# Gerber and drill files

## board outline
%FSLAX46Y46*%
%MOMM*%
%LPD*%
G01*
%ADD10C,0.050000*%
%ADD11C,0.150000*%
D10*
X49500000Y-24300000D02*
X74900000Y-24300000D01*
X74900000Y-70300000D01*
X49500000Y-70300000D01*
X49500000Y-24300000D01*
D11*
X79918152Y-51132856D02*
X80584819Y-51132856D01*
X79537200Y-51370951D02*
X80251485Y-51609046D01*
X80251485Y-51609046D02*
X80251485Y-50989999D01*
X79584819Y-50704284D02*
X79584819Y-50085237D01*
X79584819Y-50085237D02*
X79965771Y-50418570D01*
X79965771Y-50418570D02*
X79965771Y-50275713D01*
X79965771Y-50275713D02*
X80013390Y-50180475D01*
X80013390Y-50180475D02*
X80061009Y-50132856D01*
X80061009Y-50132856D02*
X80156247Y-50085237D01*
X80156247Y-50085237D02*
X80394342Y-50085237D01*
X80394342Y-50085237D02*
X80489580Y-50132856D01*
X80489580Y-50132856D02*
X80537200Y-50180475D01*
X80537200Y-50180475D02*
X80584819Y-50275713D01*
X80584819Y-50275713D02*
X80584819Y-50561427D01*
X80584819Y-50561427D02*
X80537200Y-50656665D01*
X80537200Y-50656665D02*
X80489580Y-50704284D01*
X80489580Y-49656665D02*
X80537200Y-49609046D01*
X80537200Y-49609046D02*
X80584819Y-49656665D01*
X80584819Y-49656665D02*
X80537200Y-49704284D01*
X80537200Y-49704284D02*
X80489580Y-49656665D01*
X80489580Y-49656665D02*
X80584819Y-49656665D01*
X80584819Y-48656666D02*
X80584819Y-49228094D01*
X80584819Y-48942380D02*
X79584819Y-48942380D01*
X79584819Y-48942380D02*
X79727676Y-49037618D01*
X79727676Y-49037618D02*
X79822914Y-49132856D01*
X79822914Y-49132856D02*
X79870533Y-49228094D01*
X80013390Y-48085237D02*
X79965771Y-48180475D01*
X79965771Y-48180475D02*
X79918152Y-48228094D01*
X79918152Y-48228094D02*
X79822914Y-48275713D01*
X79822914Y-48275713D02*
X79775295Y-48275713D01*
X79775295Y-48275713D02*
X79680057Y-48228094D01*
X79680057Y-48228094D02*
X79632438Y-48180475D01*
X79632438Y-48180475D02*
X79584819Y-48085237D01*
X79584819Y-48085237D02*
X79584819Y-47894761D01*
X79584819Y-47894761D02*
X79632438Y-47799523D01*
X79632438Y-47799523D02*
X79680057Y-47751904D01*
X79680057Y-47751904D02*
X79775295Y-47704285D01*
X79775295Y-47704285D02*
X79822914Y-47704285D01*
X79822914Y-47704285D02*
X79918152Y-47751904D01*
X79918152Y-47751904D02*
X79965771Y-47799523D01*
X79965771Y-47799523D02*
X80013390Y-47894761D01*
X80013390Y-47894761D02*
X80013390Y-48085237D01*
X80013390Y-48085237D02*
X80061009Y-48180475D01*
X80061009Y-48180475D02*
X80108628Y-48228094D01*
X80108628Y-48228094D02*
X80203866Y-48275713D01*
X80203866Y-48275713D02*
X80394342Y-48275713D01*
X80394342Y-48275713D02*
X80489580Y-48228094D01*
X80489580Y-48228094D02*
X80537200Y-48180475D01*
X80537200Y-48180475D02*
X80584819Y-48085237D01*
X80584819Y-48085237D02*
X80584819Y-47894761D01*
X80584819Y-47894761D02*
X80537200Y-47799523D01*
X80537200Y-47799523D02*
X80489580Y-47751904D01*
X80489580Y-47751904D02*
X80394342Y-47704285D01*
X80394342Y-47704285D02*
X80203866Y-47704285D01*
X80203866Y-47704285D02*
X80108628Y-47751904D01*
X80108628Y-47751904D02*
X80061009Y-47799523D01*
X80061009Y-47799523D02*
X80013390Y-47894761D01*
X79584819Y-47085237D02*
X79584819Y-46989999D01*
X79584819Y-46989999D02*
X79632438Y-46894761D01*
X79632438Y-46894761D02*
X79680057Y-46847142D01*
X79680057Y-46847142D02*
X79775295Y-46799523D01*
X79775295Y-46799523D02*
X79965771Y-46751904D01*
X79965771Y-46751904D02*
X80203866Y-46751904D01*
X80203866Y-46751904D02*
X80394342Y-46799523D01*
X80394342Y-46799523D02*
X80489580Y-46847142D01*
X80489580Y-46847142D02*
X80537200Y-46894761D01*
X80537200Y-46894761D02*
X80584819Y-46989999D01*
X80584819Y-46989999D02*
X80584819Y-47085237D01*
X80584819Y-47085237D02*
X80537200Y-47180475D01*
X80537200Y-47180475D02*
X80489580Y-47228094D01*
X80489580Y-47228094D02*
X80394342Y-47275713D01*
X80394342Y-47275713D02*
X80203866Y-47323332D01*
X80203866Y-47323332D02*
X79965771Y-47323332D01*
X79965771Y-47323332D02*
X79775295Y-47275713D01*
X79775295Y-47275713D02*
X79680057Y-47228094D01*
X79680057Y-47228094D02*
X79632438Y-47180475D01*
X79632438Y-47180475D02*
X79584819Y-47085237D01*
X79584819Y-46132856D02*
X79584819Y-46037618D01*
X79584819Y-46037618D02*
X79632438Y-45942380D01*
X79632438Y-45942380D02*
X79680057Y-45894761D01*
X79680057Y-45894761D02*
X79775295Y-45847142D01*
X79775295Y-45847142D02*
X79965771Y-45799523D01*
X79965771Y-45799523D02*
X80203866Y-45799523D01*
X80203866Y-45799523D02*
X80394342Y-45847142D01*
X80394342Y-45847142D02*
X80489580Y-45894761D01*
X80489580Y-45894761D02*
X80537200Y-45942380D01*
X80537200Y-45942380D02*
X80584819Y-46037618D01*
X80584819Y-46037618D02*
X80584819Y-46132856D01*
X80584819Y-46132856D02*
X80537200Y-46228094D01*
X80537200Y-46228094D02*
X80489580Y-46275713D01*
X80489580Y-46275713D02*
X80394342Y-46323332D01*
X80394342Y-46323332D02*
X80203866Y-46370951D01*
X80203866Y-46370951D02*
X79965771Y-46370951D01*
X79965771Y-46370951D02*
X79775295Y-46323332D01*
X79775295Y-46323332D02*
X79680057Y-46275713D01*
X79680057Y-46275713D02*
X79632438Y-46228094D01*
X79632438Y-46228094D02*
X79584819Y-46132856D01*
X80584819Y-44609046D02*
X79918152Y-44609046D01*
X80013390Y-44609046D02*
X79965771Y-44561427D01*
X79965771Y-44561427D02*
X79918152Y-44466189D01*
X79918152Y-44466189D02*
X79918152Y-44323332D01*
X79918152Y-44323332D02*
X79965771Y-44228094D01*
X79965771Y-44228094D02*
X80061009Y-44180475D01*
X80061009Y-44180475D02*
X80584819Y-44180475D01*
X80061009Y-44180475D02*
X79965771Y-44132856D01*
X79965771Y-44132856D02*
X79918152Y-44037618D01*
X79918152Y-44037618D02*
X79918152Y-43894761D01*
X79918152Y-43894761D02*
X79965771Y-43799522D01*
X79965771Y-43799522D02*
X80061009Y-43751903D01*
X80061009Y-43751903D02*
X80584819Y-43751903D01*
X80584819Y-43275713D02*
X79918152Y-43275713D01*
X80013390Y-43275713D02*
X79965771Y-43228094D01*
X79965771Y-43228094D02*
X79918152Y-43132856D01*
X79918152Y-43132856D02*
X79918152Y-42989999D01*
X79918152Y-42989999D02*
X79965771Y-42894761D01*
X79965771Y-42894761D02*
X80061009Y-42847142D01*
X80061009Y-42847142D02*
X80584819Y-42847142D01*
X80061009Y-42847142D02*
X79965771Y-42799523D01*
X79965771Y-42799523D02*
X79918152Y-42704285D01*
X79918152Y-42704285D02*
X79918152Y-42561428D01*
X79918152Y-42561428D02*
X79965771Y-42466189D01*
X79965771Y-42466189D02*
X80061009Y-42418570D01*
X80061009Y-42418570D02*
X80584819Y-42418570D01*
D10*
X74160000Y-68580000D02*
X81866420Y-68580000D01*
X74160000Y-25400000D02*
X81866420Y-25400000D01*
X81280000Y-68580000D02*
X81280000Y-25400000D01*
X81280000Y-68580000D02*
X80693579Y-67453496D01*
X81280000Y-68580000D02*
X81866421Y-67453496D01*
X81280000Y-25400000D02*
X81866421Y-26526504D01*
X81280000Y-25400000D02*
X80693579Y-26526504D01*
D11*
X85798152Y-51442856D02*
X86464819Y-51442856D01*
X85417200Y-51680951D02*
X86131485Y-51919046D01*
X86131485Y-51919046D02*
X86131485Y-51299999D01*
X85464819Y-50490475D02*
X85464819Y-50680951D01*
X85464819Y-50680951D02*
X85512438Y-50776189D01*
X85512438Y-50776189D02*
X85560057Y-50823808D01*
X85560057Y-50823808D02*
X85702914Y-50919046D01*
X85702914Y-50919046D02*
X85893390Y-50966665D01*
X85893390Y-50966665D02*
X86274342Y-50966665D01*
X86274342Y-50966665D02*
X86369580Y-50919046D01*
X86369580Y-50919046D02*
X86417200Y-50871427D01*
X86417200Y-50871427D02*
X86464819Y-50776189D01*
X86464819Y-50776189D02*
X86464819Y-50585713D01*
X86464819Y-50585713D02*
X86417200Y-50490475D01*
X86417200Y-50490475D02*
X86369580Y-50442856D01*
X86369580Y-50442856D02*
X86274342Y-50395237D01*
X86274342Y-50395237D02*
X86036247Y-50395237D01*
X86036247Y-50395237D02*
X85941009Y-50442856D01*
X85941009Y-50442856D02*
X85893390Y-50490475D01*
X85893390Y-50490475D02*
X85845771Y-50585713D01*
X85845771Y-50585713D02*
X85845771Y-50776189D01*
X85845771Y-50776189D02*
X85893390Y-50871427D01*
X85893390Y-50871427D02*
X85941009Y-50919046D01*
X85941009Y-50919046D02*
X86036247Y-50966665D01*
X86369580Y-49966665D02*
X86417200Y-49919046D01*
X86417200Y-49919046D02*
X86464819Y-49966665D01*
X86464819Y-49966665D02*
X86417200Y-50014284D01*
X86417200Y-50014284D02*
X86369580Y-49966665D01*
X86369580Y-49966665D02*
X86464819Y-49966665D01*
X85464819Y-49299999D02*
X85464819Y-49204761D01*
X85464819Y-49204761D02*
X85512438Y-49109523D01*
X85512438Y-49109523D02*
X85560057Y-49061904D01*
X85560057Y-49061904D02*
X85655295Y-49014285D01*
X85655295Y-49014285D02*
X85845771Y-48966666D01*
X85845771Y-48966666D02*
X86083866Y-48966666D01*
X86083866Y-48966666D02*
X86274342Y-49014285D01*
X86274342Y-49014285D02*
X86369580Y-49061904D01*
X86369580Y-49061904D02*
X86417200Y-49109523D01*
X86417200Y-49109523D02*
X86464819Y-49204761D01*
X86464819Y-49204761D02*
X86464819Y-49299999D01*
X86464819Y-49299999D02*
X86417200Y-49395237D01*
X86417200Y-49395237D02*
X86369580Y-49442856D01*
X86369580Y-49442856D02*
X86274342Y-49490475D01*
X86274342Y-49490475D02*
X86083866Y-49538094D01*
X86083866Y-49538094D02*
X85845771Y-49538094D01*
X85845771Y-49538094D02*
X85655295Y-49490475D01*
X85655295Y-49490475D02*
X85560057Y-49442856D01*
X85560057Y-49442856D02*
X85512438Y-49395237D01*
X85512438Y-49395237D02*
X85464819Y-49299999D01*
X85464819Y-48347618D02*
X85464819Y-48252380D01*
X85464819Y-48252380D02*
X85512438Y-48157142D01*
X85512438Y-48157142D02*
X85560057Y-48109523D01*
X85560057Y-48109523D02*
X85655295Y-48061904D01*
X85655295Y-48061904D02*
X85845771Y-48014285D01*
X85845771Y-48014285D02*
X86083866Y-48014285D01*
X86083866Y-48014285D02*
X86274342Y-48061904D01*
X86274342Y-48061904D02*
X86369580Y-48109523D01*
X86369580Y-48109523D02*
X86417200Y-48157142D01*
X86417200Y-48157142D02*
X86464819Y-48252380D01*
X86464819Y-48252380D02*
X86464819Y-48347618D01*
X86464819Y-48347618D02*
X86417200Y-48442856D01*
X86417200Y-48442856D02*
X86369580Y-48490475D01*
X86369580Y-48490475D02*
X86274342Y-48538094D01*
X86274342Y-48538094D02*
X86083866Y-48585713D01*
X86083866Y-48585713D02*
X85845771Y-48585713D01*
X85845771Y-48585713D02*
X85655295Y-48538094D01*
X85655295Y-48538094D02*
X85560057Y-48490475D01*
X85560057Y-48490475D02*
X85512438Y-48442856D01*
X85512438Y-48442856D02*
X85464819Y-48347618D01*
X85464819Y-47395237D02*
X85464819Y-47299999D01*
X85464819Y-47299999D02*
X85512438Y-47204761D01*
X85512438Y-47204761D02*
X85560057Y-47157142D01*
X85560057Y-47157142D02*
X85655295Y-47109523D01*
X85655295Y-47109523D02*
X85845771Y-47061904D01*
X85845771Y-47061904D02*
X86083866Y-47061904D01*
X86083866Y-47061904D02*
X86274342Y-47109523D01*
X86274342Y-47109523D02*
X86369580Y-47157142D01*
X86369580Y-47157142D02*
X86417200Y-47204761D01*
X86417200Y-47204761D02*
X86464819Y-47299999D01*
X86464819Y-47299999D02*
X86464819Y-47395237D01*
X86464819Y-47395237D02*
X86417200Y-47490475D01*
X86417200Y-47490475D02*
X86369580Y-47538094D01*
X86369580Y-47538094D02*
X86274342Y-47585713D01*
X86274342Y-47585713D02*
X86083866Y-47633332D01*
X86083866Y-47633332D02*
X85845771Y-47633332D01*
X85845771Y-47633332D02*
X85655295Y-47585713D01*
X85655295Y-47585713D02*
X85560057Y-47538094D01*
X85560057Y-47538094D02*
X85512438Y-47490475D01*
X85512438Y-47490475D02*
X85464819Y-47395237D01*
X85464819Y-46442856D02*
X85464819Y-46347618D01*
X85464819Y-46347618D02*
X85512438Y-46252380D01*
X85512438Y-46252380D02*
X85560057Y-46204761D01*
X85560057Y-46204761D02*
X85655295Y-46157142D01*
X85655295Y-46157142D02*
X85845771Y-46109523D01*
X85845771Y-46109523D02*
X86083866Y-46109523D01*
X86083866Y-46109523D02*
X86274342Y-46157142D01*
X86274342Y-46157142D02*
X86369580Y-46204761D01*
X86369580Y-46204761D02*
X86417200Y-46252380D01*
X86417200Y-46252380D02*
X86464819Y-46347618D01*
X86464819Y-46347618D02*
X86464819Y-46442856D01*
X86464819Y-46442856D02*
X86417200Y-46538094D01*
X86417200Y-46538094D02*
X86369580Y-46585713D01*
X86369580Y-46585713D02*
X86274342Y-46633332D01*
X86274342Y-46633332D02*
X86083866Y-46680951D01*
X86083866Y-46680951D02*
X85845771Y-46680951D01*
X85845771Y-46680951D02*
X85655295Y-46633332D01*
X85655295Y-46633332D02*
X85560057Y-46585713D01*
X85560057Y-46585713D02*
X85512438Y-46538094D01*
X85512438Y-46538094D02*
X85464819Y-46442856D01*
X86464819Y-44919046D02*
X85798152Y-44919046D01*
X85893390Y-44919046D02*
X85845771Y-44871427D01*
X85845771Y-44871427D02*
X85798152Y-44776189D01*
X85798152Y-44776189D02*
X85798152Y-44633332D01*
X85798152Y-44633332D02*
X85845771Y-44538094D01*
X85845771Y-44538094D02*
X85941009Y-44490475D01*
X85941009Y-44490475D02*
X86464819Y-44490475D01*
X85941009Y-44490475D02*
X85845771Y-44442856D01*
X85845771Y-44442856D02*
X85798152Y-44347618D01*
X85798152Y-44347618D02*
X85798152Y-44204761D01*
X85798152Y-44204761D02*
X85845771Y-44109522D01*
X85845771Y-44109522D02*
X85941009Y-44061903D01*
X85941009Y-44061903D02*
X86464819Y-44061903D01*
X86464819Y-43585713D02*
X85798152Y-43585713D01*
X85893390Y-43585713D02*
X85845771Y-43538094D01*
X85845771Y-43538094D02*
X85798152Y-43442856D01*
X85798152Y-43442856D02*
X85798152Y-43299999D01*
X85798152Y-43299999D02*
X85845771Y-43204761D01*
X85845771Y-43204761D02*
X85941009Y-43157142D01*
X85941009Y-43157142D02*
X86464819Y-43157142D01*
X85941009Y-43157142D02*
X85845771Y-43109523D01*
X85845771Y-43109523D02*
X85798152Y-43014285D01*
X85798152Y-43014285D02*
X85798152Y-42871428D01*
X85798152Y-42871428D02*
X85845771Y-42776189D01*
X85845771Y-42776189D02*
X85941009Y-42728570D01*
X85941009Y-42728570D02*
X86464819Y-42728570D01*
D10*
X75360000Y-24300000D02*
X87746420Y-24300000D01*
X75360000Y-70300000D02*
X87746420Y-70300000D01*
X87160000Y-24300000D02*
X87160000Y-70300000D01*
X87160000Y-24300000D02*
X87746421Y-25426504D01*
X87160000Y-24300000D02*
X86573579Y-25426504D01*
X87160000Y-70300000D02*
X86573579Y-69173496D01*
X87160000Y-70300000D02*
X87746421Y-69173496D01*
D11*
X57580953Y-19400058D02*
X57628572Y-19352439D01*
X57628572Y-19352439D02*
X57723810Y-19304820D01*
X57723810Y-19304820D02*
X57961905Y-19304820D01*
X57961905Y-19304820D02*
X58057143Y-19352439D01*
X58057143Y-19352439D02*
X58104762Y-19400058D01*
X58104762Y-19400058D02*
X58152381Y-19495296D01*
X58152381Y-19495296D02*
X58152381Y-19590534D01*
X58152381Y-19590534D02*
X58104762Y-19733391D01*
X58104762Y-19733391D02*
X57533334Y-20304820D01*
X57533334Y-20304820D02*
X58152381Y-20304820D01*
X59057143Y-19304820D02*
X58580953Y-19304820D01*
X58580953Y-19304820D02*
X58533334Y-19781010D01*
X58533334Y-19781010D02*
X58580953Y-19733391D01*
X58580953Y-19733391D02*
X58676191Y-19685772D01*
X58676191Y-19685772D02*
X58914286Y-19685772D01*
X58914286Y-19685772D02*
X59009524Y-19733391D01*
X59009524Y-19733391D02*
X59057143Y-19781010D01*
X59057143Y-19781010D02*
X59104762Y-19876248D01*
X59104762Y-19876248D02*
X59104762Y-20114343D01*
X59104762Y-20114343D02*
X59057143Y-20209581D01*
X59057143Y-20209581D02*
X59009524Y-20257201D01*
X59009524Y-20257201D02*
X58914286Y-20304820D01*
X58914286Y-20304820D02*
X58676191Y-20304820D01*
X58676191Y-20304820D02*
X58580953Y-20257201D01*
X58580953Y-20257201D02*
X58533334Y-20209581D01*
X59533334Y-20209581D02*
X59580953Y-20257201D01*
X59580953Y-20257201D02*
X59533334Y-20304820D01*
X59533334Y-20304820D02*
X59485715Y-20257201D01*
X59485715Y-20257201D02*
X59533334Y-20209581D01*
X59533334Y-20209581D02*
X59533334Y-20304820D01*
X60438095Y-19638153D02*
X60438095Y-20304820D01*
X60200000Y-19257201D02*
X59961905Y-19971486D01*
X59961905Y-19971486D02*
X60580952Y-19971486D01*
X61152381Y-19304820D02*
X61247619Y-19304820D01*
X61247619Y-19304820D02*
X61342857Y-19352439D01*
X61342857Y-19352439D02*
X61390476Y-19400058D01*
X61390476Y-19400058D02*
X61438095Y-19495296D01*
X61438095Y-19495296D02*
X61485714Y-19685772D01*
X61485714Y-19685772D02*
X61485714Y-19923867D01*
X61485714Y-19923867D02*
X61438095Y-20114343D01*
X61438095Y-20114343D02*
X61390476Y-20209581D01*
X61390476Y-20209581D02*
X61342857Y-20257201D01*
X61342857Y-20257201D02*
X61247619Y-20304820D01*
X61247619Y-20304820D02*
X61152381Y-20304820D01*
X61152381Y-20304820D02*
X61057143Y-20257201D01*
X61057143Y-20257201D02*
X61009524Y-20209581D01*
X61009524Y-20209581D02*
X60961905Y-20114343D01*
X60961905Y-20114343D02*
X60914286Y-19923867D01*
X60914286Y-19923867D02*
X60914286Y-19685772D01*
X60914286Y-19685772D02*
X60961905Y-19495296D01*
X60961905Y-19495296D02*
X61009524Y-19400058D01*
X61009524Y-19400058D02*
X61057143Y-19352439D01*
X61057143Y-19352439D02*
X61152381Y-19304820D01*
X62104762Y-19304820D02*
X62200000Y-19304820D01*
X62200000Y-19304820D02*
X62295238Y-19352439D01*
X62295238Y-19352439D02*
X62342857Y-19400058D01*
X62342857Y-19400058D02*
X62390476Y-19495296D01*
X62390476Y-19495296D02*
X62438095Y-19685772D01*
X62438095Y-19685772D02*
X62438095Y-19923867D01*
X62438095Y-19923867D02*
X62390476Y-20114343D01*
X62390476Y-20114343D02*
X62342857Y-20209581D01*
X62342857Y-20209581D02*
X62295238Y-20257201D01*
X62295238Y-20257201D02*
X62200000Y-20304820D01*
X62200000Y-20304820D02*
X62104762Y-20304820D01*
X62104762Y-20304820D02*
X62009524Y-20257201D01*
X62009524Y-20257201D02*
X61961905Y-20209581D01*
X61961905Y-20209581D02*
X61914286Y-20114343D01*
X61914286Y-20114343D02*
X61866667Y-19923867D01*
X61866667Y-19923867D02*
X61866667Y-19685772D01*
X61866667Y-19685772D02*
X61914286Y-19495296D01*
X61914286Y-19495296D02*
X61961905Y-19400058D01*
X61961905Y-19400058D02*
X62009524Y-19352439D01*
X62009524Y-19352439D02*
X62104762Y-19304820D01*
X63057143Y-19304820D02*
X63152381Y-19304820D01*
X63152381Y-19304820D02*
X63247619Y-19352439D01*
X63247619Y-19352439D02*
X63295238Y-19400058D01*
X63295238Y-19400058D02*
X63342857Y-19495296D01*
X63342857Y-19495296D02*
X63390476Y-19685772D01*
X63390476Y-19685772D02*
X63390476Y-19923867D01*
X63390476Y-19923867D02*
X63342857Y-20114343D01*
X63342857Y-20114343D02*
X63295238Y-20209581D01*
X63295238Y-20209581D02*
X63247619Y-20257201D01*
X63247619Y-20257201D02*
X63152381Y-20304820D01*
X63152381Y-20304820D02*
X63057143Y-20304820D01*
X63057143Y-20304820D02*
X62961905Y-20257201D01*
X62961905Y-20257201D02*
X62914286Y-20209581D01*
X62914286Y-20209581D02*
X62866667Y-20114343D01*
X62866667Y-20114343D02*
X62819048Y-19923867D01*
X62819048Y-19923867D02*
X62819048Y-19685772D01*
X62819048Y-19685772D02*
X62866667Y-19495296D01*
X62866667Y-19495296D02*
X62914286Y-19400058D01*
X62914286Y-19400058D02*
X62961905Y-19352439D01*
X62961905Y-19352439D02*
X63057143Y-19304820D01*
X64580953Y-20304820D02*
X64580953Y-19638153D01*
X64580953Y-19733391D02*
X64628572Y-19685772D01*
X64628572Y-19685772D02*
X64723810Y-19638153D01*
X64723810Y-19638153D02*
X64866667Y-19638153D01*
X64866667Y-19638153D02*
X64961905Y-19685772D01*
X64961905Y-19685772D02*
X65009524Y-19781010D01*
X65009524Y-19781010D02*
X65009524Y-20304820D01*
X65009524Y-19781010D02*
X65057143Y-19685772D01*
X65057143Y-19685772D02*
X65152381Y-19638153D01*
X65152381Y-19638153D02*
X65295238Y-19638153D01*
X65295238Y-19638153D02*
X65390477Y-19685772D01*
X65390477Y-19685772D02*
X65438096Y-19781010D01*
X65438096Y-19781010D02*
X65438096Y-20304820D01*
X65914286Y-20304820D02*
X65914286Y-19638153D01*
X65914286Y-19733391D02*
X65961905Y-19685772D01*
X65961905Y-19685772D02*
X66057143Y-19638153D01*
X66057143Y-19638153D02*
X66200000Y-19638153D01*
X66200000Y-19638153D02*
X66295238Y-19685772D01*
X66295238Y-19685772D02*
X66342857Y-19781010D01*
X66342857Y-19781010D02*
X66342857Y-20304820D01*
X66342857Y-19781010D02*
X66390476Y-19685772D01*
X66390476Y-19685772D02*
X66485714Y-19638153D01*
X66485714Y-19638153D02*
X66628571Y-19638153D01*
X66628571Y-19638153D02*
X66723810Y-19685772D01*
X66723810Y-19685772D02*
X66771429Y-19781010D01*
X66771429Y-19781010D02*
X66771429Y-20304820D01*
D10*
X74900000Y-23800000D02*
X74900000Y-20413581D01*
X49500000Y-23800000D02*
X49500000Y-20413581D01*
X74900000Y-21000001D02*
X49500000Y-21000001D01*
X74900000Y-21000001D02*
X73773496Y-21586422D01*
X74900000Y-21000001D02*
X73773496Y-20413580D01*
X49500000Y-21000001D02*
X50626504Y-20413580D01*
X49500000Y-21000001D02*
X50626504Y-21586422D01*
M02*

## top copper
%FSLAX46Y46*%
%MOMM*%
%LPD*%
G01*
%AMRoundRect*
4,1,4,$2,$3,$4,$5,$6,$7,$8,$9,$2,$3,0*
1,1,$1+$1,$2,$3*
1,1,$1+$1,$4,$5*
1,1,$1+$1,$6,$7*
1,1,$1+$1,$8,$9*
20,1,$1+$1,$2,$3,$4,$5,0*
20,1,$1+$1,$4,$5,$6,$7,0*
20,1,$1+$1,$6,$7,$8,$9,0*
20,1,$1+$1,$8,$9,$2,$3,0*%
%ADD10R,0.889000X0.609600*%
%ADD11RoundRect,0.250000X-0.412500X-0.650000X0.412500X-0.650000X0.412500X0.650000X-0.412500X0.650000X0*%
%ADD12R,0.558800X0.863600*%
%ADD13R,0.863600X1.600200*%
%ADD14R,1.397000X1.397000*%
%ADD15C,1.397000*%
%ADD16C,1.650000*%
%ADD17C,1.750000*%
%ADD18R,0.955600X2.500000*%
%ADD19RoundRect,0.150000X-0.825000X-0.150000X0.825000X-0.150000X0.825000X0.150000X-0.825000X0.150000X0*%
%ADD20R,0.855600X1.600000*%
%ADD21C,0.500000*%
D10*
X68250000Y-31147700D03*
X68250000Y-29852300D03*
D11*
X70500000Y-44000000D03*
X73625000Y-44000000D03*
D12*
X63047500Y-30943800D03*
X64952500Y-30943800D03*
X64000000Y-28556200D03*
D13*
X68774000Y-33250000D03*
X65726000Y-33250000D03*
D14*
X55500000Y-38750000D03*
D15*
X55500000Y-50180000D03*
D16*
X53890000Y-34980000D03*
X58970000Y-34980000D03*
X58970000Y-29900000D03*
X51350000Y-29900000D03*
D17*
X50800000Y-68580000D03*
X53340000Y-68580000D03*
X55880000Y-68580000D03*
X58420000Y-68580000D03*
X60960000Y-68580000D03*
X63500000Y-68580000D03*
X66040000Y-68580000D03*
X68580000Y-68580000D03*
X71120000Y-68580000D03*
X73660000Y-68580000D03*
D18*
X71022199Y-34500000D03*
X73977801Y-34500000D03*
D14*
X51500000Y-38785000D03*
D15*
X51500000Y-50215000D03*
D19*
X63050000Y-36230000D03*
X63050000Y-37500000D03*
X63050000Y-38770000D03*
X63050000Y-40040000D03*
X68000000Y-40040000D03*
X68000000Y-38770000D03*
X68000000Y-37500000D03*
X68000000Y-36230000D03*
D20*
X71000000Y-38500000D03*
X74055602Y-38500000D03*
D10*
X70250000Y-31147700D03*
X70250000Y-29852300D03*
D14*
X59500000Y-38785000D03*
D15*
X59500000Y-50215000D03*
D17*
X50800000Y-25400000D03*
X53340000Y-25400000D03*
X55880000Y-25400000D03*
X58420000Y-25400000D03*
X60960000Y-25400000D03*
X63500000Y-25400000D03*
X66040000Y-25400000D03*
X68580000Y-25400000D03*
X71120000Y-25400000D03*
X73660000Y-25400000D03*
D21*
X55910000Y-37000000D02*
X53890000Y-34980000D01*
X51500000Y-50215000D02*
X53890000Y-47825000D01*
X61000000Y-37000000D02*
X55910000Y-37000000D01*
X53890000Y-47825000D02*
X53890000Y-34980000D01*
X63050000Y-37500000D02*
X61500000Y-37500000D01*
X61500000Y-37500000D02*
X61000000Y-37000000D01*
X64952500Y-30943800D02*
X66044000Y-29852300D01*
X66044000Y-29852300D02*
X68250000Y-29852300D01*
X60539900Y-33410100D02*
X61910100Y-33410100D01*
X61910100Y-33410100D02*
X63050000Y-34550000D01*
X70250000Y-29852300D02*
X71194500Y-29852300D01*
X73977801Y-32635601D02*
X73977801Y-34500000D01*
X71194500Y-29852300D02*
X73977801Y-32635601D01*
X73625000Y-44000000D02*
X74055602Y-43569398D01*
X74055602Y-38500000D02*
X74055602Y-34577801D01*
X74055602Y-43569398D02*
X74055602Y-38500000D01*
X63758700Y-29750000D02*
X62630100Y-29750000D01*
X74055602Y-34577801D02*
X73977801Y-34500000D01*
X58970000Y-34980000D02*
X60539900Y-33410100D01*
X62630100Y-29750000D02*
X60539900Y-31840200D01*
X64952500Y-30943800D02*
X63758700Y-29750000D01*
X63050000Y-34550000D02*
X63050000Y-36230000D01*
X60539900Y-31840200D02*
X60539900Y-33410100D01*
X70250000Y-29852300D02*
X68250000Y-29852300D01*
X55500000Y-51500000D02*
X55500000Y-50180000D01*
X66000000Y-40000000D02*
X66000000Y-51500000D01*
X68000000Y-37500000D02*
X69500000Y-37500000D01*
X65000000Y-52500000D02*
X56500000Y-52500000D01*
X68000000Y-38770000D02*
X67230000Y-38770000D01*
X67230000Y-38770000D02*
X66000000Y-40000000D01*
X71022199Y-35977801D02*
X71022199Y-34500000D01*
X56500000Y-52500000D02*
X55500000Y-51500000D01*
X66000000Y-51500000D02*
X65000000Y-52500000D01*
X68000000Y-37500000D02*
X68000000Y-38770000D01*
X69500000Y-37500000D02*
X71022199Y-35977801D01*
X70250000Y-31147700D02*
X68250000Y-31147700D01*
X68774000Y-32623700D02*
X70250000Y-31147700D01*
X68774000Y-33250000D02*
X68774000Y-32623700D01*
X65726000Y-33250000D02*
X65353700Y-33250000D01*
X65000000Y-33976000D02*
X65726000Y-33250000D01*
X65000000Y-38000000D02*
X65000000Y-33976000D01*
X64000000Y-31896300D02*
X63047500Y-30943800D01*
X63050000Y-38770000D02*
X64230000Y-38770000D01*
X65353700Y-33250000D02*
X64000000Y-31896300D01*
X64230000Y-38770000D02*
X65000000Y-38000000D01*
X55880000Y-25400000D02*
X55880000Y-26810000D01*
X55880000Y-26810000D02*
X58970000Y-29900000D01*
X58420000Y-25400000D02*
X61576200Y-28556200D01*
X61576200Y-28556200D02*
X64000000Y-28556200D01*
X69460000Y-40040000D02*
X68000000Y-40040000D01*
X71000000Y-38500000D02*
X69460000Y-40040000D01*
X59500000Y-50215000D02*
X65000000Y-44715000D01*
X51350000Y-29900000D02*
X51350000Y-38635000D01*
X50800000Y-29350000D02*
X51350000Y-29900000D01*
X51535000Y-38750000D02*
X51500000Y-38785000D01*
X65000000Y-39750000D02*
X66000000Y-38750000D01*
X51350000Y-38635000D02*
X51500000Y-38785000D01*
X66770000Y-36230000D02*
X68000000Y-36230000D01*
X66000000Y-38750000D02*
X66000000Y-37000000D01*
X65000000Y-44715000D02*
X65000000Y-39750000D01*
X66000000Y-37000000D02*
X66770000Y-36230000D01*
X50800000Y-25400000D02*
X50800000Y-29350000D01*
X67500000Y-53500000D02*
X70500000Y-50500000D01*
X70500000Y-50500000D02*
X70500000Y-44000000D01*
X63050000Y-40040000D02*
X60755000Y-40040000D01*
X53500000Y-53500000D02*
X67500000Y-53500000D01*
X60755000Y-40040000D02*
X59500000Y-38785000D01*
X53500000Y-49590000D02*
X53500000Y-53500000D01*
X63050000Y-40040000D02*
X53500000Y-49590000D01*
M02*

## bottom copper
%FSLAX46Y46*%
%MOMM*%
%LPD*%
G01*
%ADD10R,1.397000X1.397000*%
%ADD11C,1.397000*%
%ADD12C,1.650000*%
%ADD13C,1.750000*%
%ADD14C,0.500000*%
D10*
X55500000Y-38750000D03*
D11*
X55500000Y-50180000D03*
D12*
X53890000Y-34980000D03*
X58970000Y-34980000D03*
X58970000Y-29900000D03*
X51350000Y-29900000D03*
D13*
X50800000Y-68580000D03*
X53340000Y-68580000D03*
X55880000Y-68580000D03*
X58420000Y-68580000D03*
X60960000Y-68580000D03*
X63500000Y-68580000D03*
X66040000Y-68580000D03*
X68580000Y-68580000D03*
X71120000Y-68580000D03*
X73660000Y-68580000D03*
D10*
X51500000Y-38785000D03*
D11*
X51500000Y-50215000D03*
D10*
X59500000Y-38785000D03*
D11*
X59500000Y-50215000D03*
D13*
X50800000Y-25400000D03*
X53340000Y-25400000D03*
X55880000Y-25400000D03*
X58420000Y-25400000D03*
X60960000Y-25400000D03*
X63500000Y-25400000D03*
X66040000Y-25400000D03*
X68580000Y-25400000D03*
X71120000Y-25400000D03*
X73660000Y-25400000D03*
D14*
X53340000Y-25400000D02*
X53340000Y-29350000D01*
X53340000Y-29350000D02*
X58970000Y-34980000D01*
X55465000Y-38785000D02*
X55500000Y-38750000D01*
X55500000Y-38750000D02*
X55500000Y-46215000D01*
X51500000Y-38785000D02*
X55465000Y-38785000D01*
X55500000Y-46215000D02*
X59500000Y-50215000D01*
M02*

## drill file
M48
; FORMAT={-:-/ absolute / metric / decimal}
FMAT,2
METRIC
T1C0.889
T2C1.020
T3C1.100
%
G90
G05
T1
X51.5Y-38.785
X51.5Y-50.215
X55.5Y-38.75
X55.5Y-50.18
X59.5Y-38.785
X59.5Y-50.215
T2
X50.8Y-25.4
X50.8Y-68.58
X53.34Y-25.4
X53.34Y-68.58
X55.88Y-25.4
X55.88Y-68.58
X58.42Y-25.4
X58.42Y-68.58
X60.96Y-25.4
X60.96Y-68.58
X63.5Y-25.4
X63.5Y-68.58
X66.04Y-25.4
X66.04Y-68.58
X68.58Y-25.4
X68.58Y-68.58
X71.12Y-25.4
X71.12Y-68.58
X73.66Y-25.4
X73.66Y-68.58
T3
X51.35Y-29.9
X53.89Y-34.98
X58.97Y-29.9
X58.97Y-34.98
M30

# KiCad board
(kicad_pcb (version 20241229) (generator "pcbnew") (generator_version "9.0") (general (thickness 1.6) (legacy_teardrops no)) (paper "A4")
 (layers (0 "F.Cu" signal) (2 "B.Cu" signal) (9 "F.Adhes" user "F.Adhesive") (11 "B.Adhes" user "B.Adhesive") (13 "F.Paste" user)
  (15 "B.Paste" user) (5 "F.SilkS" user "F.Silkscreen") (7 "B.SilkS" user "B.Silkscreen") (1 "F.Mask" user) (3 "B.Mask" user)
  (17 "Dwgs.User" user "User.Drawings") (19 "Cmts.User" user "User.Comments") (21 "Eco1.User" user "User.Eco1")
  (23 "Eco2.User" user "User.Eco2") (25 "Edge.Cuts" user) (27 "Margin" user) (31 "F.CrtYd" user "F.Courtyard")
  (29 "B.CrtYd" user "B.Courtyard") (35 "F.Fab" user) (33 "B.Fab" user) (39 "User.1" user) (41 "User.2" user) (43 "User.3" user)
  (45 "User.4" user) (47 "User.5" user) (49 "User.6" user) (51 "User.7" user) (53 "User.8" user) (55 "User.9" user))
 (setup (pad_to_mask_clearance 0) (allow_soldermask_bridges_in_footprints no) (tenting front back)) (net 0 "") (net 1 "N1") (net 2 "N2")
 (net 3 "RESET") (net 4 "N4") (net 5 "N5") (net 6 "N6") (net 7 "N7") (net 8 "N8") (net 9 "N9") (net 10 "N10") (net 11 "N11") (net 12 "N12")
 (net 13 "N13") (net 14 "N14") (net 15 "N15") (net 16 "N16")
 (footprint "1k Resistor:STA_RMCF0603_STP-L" (layer "F.Cu") (at 68.25 30.5 90)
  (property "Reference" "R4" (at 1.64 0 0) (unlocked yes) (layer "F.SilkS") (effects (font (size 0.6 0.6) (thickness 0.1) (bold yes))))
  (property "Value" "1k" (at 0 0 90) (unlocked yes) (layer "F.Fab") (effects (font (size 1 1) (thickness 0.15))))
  (pad "1" smd rect (at -0.6477 0 90) (size 0.6096 0.889) (layers "F.Cu" "F.Mask" "F.Paste") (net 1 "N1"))
  (pad "2" smd rect (at 0.6477 0 90) (size 0.6096 0.889) (layers "F.Cu" "F.Mask" "F.Paste") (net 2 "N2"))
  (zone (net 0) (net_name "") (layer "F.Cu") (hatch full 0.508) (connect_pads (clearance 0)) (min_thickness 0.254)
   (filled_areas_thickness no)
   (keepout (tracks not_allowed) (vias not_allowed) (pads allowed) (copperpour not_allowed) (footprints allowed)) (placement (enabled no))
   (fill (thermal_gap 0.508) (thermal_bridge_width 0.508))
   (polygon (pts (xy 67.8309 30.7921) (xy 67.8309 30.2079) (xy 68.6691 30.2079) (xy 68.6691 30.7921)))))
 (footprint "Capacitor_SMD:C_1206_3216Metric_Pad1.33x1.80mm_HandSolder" (layer "F.Cu") (at 72.0625 44)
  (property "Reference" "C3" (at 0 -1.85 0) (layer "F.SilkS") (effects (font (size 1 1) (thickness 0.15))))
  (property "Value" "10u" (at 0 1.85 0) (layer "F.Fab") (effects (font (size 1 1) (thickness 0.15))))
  (pad "1" smd roundrect (at -1.5625 0) (size 1.325 1.8) (layers "F.Cu" "F.Mask" "F.Paste") (roundrect_rratio 0.188679) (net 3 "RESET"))
  (pad "2" smd roundrect (at 1.5625 0) (size 1.325 1.8) (layers "F.Cu" "F.Mask" "F.Paste") (roundrect_rratio 0.188679) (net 2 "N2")))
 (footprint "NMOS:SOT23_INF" (layer "F.Cu") (at 64 29.75)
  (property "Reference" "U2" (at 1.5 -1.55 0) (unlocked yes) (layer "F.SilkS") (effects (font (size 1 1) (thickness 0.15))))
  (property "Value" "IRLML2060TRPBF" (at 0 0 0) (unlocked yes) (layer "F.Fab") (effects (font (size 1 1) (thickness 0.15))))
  (pad "1" smd rect (at -0.9525 1.1938) (size 0.5588 0.8636) (layers "F.Cu" "F.Mask" "F.Paste") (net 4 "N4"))
  (pad "2" smd rect (at 0.9525 1.1938) (size 0.5588 0.8636) (layers "F.Cu" "F.Mask" "F.Paste") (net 2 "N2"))
  (pad "3" smd rect (at 0 -1.1938) (size 0.5588 0.8636) (layers "F.Cu" "F.Mask" "F.Paste") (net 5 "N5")))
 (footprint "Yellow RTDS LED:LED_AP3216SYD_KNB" (layer "F.Cu") (at 67.25 33.25 180)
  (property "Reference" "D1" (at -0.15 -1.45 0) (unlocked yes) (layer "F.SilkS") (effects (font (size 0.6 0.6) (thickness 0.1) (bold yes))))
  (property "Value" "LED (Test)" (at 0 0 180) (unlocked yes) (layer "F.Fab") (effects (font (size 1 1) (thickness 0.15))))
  (pad "1" smd rect (at -1.524 0 180) (size 0.8636 1.6002) (layers "F.Cu" "F.Mask" "F.Paste") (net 1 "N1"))
  (pad "2" smd rect (at 1.524 0 180) (size 0.8636 1.6002) (layers "F.Cu" "F.Mask" "F.Paste") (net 4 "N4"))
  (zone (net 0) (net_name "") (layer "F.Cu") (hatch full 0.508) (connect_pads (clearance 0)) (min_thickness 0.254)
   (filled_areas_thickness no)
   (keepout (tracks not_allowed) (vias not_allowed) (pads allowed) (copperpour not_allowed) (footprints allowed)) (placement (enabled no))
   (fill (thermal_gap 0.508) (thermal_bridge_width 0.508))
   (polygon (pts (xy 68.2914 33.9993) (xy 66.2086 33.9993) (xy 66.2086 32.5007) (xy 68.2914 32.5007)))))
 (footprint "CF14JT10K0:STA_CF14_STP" (layer "F.Cu") (at 55.5 38.75 -90)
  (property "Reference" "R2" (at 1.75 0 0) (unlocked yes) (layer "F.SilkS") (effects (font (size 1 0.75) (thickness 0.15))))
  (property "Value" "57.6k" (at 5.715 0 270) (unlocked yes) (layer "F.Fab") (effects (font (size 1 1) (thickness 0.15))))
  (pad "1" thru_hole rect (at 0 0 270) (size 1.397 1.397) (drill 0.889) (layers "*.Cu" "*.Mask") (remove_unused_layers no) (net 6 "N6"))
  (pad "2" thru_hole circle (at 11.43 0 270) (size 1.397 1.397) (drill 0.889) (layers "*.Cu" "*.Mask") (remove_unused_layers no)
   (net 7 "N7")))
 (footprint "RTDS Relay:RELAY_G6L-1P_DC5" (layer "F.Cu") (at 55.16 32.44)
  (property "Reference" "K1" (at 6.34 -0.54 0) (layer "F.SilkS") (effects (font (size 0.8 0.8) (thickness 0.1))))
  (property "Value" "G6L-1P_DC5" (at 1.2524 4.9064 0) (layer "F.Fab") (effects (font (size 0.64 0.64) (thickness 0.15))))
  (pad "2" thru_hole circle (at -1.27 2.54) (size 1.65 1.65) (drill 1.1) (layers "*.Cu" "*.Mask") (remove_unused_layers no) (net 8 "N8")
   (solder_mask_margin 0.102))
  (pad "4" thru_hole circle (at 3.81 2.54) (size 1.65 1.65) (drill 1.1) (layers "*.Cu" "*.Mask") (remove_unused_layers no) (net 2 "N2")
   (solder_mask_margin 0.102))
  (pad "5" thru_hole circle (at 3.81 -2.54) (size 1.65 1.65) (drill 1.1) (layers "*.Cu" "*.Mask") (remove_unused_layers no) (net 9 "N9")
   (solder_mask_margin 0.102))
  (pad "8" thru_hole circle (at -3.81 -2.54) (size 1.65 1.65) (drill 1.1) (layers "*.Cu" "*.Mask") (remove_unused_layers no) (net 6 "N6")
   (solder_mask_margin 0.102)))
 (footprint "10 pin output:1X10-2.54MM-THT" (layer "F.Cu") (at 50.8 68.58)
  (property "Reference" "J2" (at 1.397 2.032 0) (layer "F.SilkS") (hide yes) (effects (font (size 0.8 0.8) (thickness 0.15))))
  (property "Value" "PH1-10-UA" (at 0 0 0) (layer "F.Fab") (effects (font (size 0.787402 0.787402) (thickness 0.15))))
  (pad "1" thru_hole circle (at 0 0) (size 1.75 1.75) (drill 1.02) (layers "*.Cu" "*.Mask") (remove_unused_layers no)
   (solder_mask_margin 0.102))
  (pad "2" thru_hole circle (at 2.54 0) (size 1.75 1.75) (drill 1.02) (layers "*.Cu" "*.Mask") (remove_unused_layers no)
   (solder_mask_margin 0.102))
  (pad "3" thru_hole circle (at 5.08 0) (size 1.75 1.75) (drill 1.02) (layers "*.Cu" "*.Mask") (remove_unused_layers no)
   (solder_mask_margin 0.102))
  (pad "4" thru_hole circle (at 7.62 0) (size 1.75 1.75) (drill 1.02) (layers "*.Cu" "*.Mask") (remove_unused_layers no)
   (solder_mask_margin 0.102))
  (pad "5" thru_hole circle (at 10.16 0) (size 1.75 1.75) (drill 1.02) (layers "*.Cu" "*.Mask") (remove_unused_layers no)
   (solder_mask_margin 0.102))
  (pad "6" thru_hole circle (at 12.7 0) (size 1.75 1.75) (drill 1.02) (layers "*.Cu" "*.Mask") (remove_unused_layers no)
   (solder_mask_margin 0.102))
  (pad "7" thru_hole circle (at 15.24 0) (size 1.75 1.75) (drill 1.02) (layers "*.Cu" "*.Mask") (remove_unused_layers no)
   (solder_mask_margin 0.102))
  (pad "8" thru_hole circle (at 17.78 0) (size 1.75 1.75) (drill 1.02) (layers "*.Cu" "*.Mask") (remove_unused_layers no)
   (solder_mask_margin 0.102))
  (pad "9" thru_hole circle (at 20.32 0) (size 1.75 1.75) (drill 1.02) (layers "*.Cu" "*.Mask") (remove_unused_layers no)
   (solder_mask_margin 0.102))
  (pad "10" thru_hole circle (at 22.86 0) (size 1.75 1.75) (drill 1.02) (layers "*.Cu" "*.Mask") (remove_unused_layers no)
   (solder_mask_margin 0.102)))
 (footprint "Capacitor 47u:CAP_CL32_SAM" (layer "F.Cu") (at 72.5 34.5)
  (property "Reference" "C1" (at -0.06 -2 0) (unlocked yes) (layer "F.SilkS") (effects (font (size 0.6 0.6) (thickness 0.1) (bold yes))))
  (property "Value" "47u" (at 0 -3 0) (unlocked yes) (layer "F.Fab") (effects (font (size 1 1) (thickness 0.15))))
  (pad "1" smd rect (at -1.477801 0) (size 0.9556 2.5) (layers "F.Cu" "F.Mask" "F.Paste") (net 7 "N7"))
  (pad "2" smd rect (at 1.477801 0) (size 0.9556 2.5) (layers "F.Cu" "F.Mask" "F.Paste") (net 2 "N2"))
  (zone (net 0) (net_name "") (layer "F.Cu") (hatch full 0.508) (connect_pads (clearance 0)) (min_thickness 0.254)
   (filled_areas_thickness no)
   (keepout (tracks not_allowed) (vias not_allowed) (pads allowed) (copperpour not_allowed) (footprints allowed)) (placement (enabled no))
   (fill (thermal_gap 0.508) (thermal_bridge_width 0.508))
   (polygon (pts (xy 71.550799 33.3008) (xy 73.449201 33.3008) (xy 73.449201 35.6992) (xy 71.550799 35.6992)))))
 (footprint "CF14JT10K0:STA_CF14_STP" (layer "F.Cu") (at 51.5 38.785 -90)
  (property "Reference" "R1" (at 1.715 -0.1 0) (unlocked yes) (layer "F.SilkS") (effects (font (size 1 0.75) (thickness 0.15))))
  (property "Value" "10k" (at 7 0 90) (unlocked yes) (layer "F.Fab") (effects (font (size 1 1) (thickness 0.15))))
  (pad "1" thru_hole rect (at 0 0 270) (size 1.397 1.397) (drill 0.889) (layers "*.Cu" "*.Mask") (remove_unused_layers no) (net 6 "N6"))
  (pad "2" thru_hole circle (at 11.43 0 270) (size 1.397 1.397) (drill 0.889) (layers "*.Cu" "*.Mask") (remove_unused_layers no)
   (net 8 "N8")))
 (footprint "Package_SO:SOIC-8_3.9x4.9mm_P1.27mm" (layer "F.Cu") (at 65.525 38.135)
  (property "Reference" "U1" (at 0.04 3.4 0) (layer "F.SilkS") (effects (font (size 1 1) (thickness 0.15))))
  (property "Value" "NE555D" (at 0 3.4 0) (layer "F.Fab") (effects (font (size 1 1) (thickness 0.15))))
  (pad "1" smd roundrect (at -2.475 -1.905) (size 1.95 0.6) (layers "F.Cu" "F.Mask" "F.Paste") (roundrect_rratio 0.25) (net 2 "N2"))
  (pad "2" smd roundrect (at -2.475 -0.635) (size 1.95 0.6) (layers "F.Cu" "F.Mask" "F.Paste") (roundrect_rratio 0.25) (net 8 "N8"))
  (pad "3" smd roundrect (at -2.475 0.635) (size 1.95 0.6) (layers "F.Cu" "F.Mask" "F.Paste") (roundrect_rratio 0.25) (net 4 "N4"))
  (pad "4" smd roundrect (at -2.475 1.905) (size 1.95 0.6) (layers "F.Cu" "F.Mask" "F.Paste") (roundrect_rratio 0.25) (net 3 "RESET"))
  (pad "5" smd roundrect (at 2.475 1.905) (size 1.95 0.6) (layers "F.Cu" "F.Mask" "F.Paste") (roundrect_rratio 0.25) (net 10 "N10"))
  (pad "6" smd roundrect (at 2.475 0.635) (size 1.95 0.6) (layers "F.Cu" "F.Mask" "F.Paste") (roundrect_rratio 0.25) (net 7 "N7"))
  (pad "7" smd roundrect (at 2.475 -0.635) (size 1.95 0.6) (layers "F.Cu" "F.Mask" "F.Paste") (roundrect_rratio 0.25) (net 7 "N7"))
  (pad "8" smd roundrect (at 2.475 -1.905) (size 1.95 0.6) (layers "F.Cu" "F.Mask" "F.Paste") (roundrect_rratio 0.25) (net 6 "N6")))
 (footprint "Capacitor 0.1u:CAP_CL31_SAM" (layer "F.Cu") (at 72.527801 38.5)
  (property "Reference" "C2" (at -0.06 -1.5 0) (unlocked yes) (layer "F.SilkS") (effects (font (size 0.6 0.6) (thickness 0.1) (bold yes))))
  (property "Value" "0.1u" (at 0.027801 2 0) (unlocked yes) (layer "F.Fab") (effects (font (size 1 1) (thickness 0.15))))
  (pad "1" smd rect (at -1.527801 0) (size 0.8556 1.6) (layers "F.Cu" "F.Mask" "F.Paste") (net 10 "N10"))
  (pad "2" smd rect (at 1.527801 0) (size 0.8556 1.6) (layers "F.Cu" "F.Mask" "F.Paste") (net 2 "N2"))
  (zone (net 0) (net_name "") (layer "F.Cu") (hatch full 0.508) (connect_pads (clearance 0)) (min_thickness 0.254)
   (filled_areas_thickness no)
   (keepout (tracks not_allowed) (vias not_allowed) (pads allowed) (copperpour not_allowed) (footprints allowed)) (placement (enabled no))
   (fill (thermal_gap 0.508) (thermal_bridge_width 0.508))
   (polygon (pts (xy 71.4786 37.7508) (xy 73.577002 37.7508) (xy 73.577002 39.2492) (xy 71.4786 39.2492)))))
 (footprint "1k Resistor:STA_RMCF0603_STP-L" (layer "F.Cu") (at 70.25 30.5 90)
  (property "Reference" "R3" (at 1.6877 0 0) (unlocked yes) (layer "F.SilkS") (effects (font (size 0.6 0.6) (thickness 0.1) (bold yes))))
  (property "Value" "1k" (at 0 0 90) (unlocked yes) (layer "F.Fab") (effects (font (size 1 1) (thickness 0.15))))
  (pad "1" smd rect (at -0.6477 0 90) (size 0.6096 0.889) (layers "F.Cu" "F.Mask" "F.Paste") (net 1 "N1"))
  (pad "2" smd rect (at 0.6477 0 90) (size 0.6096 0.889) (layers "F.Cu" "F.Mask" "F.Paste") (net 2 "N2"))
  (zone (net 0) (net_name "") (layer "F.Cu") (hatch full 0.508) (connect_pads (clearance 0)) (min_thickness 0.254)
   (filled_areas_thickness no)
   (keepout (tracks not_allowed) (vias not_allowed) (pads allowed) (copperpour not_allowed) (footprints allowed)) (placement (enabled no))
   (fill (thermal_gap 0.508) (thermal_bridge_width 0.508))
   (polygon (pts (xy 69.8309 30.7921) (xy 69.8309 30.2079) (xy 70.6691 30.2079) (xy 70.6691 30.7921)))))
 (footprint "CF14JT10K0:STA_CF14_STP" (layer "F.Cu") (at 59.5 38.785 -90)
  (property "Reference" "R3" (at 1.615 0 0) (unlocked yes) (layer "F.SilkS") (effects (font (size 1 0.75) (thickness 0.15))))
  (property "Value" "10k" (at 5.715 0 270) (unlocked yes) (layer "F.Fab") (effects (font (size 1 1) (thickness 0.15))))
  (pad "1" thru_hole rect (at 0 0 270) (size 1.397 1.397) (drill 0.889) (layers "*.Cu" "*.Mask") (remove_unused_layers no) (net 3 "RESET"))
  (pad "2" thru_hole circle (at 11.43 0 270) (size 1.397 1.397) (drill 0.889) (layers "*.Cu" "*.Mask") (remove_unused_layers no)
   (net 6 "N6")))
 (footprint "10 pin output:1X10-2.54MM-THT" (layer "F.Cu") (at 50.8 25.4)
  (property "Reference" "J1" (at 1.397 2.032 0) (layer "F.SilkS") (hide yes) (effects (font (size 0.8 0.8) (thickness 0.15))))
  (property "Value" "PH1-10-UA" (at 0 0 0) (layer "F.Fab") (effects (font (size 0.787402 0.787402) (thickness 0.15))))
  (pad "1" thru_hole circle (at 0 0) (size 1.75 1.75) (drill 1.02) (layers "*.Cu" "*.Mask") (remove_unused_layers no) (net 6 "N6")
   (solder_mask_margin 0.102))
  (pad "2" thru_hole circle (at 2.54 0) (size 1.75 1.75) (drill 1.02) (layers "*.Cu" "*.Mask") (remove_unused_layers no) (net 2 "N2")
   (solder_mask_margin 0.102))
  (pad "3" thru_hole circle (at 5.08 0) (size 1.75 1.75) (drill 1.02) (layers "*.Cu" "*.Mask") (remove_unused_layers no) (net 9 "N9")
   (solder_mask_margin 0.102))
  (pad "4" thru_hole circle (at 7.62 0) (size 1.75 1.75) (drill 1.02) (layers "*.Cu" "*.Mask") (remove_unused_layers no) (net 5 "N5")
   (solder_mask_margin 0.102))
  (pad "5" thru_hole circle (at 10.16 0) (size 1.75 1.75) (drill 1.02) (layers "*.Cu" "*.Mask") (remove_unused_layers no) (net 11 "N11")
   (solder_mask_margin 0.102))
  (pad "6" thru_hole circle (at 12.7 0) (size 1.75 1.75) (drill 1.02) (layers "*.Cu" "*.Mask") (remove_unused_layers no) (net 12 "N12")
   (solder_mask_margin 0.102))
  (pad "7" thru_hole circle (at 15.24 0) (size 1.75 1.75) (drill 1.02) (layers "*.Cu" "*.Mask") (remove_unused_layers no) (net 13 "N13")
   (solder_mask_margin 0.102))
  (pad "8" thru_hole circle (at 17.78 0) (size 1.75 1.75) (drill 1.02) (layers "*.Cu" "*.Mask") (remove_unused_layers no) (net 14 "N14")
   (solder_mask_margin 0.102))
  (pad "9" thru_hole circle (at 20.32 0) (size 1.75 1.75) (drill 1.02) (layers "*.Cu" "*.Mask") (remove_unused_layers no) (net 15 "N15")
   (solder_mask_margin 0.102))
  (pad "10" thru_hole circle (at 22.86 0) (size 1.75 1.75) (drill 1.02) (layers "*.Cu" "*.Mask") (remove_unused_layers no) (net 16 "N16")
   (solder_mask_margin 0.102)))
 (gr_rect (start 49.5 24.3) (end 74.9 70.3) (stroke (width 0.05) (type default)) (fill no) (layer "Edge.Cuts"))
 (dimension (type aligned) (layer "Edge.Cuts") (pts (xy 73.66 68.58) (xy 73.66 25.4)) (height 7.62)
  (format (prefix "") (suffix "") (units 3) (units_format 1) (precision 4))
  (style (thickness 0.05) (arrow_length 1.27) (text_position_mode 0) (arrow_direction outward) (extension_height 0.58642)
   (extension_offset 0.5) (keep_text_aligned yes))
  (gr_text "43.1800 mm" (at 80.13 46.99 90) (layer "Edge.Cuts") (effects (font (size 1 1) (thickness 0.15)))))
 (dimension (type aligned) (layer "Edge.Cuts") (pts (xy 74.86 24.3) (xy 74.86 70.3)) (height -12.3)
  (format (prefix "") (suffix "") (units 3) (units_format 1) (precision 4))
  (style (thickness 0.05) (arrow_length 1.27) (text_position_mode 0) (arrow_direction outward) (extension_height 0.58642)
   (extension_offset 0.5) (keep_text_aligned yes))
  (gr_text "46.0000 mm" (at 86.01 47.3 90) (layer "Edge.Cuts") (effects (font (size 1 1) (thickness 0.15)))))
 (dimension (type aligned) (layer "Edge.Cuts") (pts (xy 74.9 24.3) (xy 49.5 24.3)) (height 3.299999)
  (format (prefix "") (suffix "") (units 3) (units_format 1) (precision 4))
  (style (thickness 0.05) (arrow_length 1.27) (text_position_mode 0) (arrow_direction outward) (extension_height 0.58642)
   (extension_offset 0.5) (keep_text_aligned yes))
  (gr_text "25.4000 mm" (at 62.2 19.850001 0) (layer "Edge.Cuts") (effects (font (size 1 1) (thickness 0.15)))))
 (segment (start 55.91 37) (end 53.89 34.98) (width 0.5) (layer "F.Cu") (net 8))
 (segment (start 51.5 50.215) (end 53.89 47.825) (width 0.5) (layer "F.Cu") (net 8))
 (segment (start 61 37) (end 55.91 37) (width 0.5) (layer "F.Cu") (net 8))
 (segment (start 53.89 47.825) (end 53.89 34.98) (width 0.5) (layer "F.Cu") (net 8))
 (segment (start 63.05 37.5) (end 61.5 37.5) (width 0.5) (layer "F.Cu") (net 8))
 (segment (start 61.5 37.5) (end 61 37) (width 0.5) (layer "F.Cu") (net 8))
 (segment (start 64.9525 30.9438) (end 66.044 29.8523) (width 0.5) (layer "F.Cu") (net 2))
 (segment (start 66.044 29.8523) (end 68.25 29.8523) (width 0.5) (layer "F.Cu") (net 2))
 (segment (start 60.5399 33.4101) (end 61.9101 33.4101) (width 0.5) (layer "F.Cu") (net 2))
 (segment (start 61.9101 33.4101) (end 63.05 34.55) (width 0.5) (layer "F.Cu") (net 2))
 (segment (start 70.25 29.8523) (end 71.1945 29.8523) (width 0.5) (layer "F.Cu") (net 2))
 (segment (start 73.977801 32.635601) (end 73.977801 34.5) (width 0.5) (layer "F.Cu") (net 2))
 (segment (start 71.1945 29.8523) (end 73.977801 32.635601) (width 0.5) (layer "F.Cu") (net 2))
 (segment (start 73.625 44) (end 74.055602 43.569398) (width 0.5) (layer "F.Cu") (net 2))
 (segment (start 74.055602 38.5) (end 74.055602 34.577801) (width 0.5) (layer "F.Cu") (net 2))
 (segment (start 74.055602 43.569398) (end 74.055602 38.5) (width 0.5) (layer "F.Cu") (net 2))
 (segment (start 63.7587 29.75) (end 62.6301 29.75) (width 0.5) (layer "F.Cu") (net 2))
 (segment (start 74.055602 34.577801) (end 73.977801 34.5) (width 0.5) (layer "F.Cu") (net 2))
 (segment (start 58.97 34.98) (end 60.5399 33.4101) (width 0.5) (layer "F.Cu") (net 2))
 (segment (start 62.6301 29.75) (end 60.5399 31.8402) (width 0.5) (layer "F.Cu") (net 2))
 (segment (start 64.9525 30.9438) (end 63.7587 29.75) (width 0.5) (layer "F.Cu") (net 2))
 (segment (start 63.05 34.55) (end 63.05 36.23) (width 0.5) (layer "F.Cu") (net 2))
 (segment (start 60.5399 31.8402) (end 60.5399 33.4101) (width 0.5) (layer "F.Cu") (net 2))
 (segment (start 70.25 29.8523) (end 68.25 29.8523) (width 0.5) (layer "F.Cu") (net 2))
 (segment (start 53.34 25.4) (end 53.34 29.35) (width 0.5) (layer "B.Cu") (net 2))
 (segment (start 53.34 29.35) (end 58.97 34.98) (width 0.5) (layer "B.Cu") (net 2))
 (segment (start 55.5 51.5) (end 55.5 50.18) (width 0.5) (layer "F.Cu") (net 7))
 (segment (start 66 40) (end 66 51.5) (width 0.5) (layer "F.Cu") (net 7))
 (segment (start 68 37.5) (end 69.5 37.5) (width 0.5) (layer "F.Cu") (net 7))
 (segment (start 65 52.5) (end 56.5 52.5) (width 0.5) (layer "F.Cu") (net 7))
 (segment (start 68 38.77) (end 67.23 38.77) (width 0.5) (layer "F.Cu") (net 7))
 (segment (start 67.23 38.77) (end 66 40) (width 0.5) (layer "F.Cu") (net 7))
 (segment (start 71.022199 35.977801) (end 71.022199 34.5) (width 0.5) (layer "F.Cu") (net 7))
 (segment (start 56.5 52.5) (end 55.5 51.5) (width 0.5) (layer "F.Cu") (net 7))
 (segment (start 66 51.5) (end 65 52.5) (width 0.5) (layer "F.Cu") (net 7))
 (segment (start 68 37.5) (end 68 38.77) (width 0.5) (layer "F.Cu") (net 7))
 (segment (start 69.5 37.5) (end 71.022199 35.977801) (width 0.5) (layer "F.Cu") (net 7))
 (segment (start 70.25 31.1477) (end 68.25 31.1477) (width 0.5) (layer "F.Cu") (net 1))
 (segment (start 68.774 32.6237) (end 70.25 31.1477) (width 0.5) (layer "F.Cu") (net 1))
 (segment (start 68.774 33.25) (end 68.774 32.6237) (width 0.5) (layer "F.Cu") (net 1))
 (segment (start 65.726 33.25) (end 65.3537 33.25) (width 0.5) (layer "F.Cu") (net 4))
 (segment (start 65 33.976) (end 65.726 33.25) (width 0.5) (layer "F.Cu") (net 4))
 (segment (start 65 38) (end 65 33.976) (width 0.5) (layer "F.Cu") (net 4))
 (segment (start 64 31.8963) (end 63.0475 30.9438) (width 0.5) (layer "F.Cu") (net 4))
 (segment (start 63.05 38.77) (end 64.23 38.77) (width 0.5) (layer "F.Cu") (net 4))
 (segment (start 65.3537 33.25) (end 64 31.8963) (width 0.5) (layer "F.Cu") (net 4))
 (segment (start 64.23 38.77) (end 65 38) (width 0.5) (layer "F.Cu") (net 4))
 (segment (start 55.88 25.4) (end 55.88 26.81) (width 0.5) (layer "F.Cu") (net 9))
 (segment (start 55.88 26.81) (end 58.97 29.9) (width 0.5) (layer "F.Cu") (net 9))
 (segment (start 58.42 25.4) (end 61.5762 28.5562) (width 0.5) (layer "F.Cu") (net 5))
 (segment (start 61.5762 28.5562) (end 64 28.5562) (width 0.5) (layer "F.Cu") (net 5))
 (segment (start 69.46 40.04) (end 68 40.04) (width 0.5) (layer "F.Cu") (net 10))
 (segment (start 71 38.5) (end 69.46 40.04) (width 0.5) (layer "F.Cu") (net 10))
 (segment (start 59.5 50.215) (end 65 44.715) (width 0.5) (layer "F.Cu") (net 6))
 (segment (start 51.35 29.9) (end 51.35 38.635) (width 0.5) (layer "F.Cu") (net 6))
 (segment (start 50.8 29.35) (end 51.35 29.9) (width 0.5) (layer "F.Cu") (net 6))
 (segment (start 51.535 38.75) (end 51.5 38.785) (width 0.5) (layer "F.Cu") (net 6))
 (segment (start 65 39.75) (end 66 38.75) (width 0.5) (layer "F.Cu") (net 6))
 (segment (start 51.35 38.635) (end 51.5 38.785) (width 0.5) (layer "F.Cu") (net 6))
 (segment (start 66.77 36.23) (end 68 36.23) (width 0.5) (layer "F.Cu") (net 6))
 (segment (start 66 38.75) (end 66 37) (width 0.5) (layer "F.Cu") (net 6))
 (segment (start 65 44.715) (end 65 39.75) (width 0.5) (layer "F.Cu") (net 6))
 (segment (start 66 37) (end 66.77 36.23) (width 0.5) (layer "F.Cu") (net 6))
 (segment (start 50.8 25.4) (end 50.8 29.35) (width 0.5) (layer "F.Cu") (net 6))
 (segment (start 55.465 38.785) (end 55.5 38.75) (width 0.5) (layer "B.Cu") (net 6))
 (segment (start 55.5 38.75) (end 55.5 46.215) (width 0.5) (layer "B.Cu") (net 6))
 (segment (start 51.5 38.785) (end 55.465 38.785) (width 0.5) (layer "B.Cu") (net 6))
 (segment (start 55.5 46.215) (end 59.5 50.215) (width 0.5) (layer "B.Cu") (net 6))
 (segment (start 67.5 53.5) (end 70.5 50.5) (width 0.5) (layer "F.Cu") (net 3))
 (segment (start 70.5 50.5) (end 70.5 44) (width 0.5) (layer "F.Cu") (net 3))
 (segment (start 63.05 40.04) (end 60.755 40.04) (width 0.5) (layer "F.Cu") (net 3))
 (segment (start 53.5 53.5) (end 67.5 53.5) (width 0.5) (layer "F.Cu") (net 3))
 (segment (start 60.755 40.04) (end 59.5 38.785) (width 0.5) (layer "F.Cu") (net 3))
 (segment (start 53.5 49.59) (end 53.5 53.5) (width 0.5) (layer "F.Cu") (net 3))
 (segment (start 63.05 40.04) (end 53.5 49.59) (width 0.5) (layer "F.Cu") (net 3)))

